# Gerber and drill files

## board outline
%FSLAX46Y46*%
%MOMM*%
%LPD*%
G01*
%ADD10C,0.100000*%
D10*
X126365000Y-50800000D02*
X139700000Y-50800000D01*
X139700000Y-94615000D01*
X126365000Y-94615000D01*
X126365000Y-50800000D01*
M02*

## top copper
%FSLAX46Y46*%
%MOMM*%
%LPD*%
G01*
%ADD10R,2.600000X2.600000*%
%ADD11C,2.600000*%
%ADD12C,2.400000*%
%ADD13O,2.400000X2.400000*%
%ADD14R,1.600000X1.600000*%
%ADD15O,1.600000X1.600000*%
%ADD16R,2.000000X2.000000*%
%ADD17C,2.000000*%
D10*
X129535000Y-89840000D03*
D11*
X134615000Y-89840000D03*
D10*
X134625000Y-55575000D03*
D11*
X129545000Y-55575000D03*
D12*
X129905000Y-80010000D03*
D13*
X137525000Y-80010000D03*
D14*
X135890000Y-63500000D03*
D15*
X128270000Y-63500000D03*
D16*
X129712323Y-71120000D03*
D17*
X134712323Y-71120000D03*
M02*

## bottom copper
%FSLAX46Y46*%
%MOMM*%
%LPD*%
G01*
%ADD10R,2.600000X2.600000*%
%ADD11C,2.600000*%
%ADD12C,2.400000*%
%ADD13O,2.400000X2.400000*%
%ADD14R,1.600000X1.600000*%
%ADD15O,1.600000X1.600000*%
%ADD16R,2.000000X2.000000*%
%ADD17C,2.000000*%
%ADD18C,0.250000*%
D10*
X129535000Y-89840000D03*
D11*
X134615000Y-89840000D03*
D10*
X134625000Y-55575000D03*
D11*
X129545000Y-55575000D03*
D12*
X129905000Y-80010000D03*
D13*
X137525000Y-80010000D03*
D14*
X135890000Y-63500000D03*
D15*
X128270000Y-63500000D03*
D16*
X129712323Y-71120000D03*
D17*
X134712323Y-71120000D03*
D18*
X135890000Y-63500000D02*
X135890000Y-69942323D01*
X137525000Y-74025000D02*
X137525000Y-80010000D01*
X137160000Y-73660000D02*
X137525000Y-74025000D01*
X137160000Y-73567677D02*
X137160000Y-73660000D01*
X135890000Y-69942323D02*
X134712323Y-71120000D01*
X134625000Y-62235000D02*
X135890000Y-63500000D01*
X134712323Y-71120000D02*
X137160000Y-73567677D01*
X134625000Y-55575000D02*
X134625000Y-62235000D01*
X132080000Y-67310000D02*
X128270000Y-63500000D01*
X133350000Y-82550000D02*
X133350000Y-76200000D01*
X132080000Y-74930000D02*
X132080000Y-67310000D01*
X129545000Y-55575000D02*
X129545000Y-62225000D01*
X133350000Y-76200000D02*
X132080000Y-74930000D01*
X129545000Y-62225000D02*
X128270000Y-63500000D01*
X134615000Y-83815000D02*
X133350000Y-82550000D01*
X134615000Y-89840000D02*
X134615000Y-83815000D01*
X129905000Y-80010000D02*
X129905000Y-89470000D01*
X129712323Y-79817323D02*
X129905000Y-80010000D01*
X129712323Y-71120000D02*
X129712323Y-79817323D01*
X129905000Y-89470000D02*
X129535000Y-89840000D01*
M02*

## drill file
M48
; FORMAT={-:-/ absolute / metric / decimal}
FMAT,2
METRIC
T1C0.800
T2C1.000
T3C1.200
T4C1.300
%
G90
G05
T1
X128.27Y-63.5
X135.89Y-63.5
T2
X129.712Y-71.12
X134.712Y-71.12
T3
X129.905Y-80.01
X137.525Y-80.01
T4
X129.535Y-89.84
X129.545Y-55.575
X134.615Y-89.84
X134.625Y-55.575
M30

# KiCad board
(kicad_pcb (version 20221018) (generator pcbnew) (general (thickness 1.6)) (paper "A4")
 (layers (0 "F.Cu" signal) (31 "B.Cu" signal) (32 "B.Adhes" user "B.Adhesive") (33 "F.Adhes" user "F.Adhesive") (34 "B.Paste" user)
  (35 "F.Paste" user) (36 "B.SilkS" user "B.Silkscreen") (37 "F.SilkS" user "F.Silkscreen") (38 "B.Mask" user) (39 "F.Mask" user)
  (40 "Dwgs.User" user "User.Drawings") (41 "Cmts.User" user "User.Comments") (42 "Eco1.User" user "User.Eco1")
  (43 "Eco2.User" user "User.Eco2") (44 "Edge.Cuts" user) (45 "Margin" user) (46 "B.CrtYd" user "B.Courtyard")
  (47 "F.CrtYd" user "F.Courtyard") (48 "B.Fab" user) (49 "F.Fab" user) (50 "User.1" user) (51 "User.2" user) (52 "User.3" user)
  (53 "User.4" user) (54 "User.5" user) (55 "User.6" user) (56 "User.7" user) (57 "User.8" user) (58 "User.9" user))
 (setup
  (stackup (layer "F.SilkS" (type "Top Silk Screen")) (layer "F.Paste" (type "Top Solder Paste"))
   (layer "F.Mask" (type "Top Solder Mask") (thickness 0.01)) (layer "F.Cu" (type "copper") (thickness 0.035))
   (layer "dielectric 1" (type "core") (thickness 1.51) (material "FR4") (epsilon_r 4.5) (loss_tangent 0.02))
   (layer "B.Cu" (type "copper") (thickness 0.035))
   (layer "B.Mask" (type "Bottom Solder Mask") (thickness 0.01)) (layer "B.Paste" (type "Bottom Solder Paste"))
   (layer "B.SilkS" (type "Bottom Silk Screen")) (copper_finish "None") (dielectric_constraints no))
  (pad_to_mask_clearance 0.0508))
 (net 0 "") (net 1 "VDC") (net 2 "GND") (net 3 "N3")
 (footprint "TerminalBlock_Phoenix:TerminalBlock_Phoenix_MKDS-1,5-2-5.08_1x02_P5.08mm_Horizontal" (layer "F.Cu") (at 129.535 89.84)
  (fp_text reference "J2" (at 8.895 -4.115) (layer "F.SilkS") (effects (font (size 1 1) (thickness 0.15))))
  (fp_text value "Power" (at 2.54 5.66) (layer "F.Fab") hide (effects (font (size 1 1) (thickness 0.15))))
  (pad "1" thru_hole rect (at 0 0) (size 2.6 2.6) (drill 1.3) (layers "*.Cu" "*.Mask") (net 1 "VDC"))
  (pad "2" thru_hole circle (at 5.08 0) (size 2.6 2.6) (drill 1.3) (layers "*.Cu" "*.Mask") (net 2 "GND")))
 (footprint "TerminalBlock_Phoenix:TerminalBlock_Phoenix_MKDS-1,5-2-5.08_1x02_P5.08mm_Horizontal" (layer "F.Cu") (at 134.625 55.575 180)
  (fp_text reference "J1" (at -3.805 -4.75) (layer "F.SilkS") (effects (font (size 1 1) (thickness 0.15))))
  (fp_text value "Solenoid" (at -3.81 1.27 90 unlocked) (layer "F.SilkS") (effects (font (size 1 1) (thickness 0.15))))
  (pad "1" thru_hole rect (at 0 0 180) (size 2.6 2.6) (drill 1.3) (layers "*.Cu" "*.Mask") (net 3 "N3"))
  (pad "2" thru_hole circle (at 5.08 0 180) (size 2.6 2.6) (drill 1.3) (layers "*.Cu" "*.Mask") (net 2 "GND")))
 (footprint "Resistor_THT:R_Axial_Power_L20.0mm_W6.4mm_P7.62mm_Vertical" (layer "F.Cu") (at 129.905 80.01)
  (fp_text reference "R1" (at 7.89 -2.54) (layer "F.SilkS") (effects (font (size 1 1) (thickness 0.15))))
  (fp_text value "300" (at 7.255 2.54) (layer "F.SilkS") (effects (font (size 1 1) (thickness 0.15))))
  (pad "1" thru_hole circle (at 0 0) (size 2.4 2.4) (drill 1.2) (layers "*.Cu" "*.Mask") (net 1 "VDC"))
  (pad "2" thru_hole oval (at 7.62 0) (size 2.4 2.4) (drill 1.2) (layers "*.Cu" "*.Mask") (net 3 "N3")))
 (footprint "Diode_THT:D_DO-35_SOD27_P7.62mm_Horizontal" (layer "F.Cu") (at 135.89 63.5 180)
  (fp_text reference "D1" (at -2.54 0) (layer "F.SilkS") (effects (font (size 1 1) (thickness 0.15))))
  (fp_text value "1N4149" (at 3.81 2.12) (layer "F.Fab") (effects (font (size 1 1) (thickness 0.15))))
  (pad "1" thru_hole rect (at 0 0 180) (size 1.6 1.6) (drill 0.8) (layers "*.Cu" "*.Mask") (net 3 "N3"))
  (pad "2" thru_hole oval (at 7.62 0 180) (size 1.6 1.6) (drill 0.8) (layers "*.Cu" "*.Mask") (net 2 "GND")))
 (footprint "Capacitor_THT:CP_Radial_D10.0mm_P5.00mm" (layer "F.Cu") (at 129.712323 71.12)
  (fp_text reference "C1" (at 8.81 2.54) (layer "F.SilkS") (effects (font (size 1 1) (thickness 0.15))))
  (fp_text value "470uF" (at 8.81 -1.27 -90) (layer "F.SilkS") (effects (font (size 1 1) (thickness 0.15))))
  (pad "1" thru_hole rect (at 0 0) (size 2 2) (drill 1) (layers "*.Cu" "*.Mask") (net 1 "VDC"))
  (pad "2" thru_hole circle (at 5 0) (size 2 2) (drill 1) (layers "*.Cu" "*.Mask") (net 3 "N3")))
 (gr_rect (start 126.365 50.8) (end 139.7 94.615) (stroke (width 0.1) (type default)) (fill none) (layer "Edge.Cuts"))
 (segment (start 135.89 63.5) (end 135.89 69.942323) (width 0.25) (layer "B.Cu") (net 3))
 (segment (start 137.525 74.025) (end 137.525 80.01) (width 0.25) (layer "B.Cu") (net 3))
 (segment (start 137.16 73.66) (end 137.525 74.025) (width 0.25) (layer "B.Cu") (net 3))
 (segment (start 137.16 73.567677) (end 137.16 73.66) (width 0.25) (layer "B.Cu") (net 3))
 (segment (start 135.89 69.942323) (end 134.712323 71.12) (width 0.25) (layer "B.Cu") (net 3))
 (segment (start 134.625 62.235) (end 135.89 63.5) (width 0.25) (layer "B.Cu") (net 3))
 (segment (start 134.712323 71.12) (end 137.16 73.567677) (width 0.25) (layer "B.Cu") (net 3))
 (segment (start 134.625 55.575) (end 134.625 62.235) (width 0.25) (layer "B.Cu") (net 3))
 (segment (start 132.08 67.31) (end 128.27 63.5) (width 0.25) (layer "B.Cu") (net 2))
 (segment (start 133.35 82.55) (end 133.35 76.2) (width 0.25) (layer "B.Cu") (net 2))
 (segment (start 132.08 74.93) (end 132.08 67.31) (width 0.25) (layer "B.Cu") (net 2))
 (segment (start 129.545 55.575) (end 129.545 62.225) (width 0.25) (layer "B.Cu") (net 2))
 (segment (start 133.35 76.2) (end 132.08 74.93) (width 0.25) (layer "B.Cu") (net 2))
 (segment (start 129.545 62.225) (end 128.27 63.5) (width 0.25) (layer "B.Cu") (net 2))
 (segment (start 134.615 83.815) (end 133.35 82.55) (width 0.25) (layer "B.Cu") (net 2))
 (segment (start 134.615 89.84) (end 134.615 83.815) (width 0.25) (layer "B.Cu") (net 2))
 (segment (start 129.905 80.01) (end 129.905 89.47) (width 0.25) (layer "B.Cu") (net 1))
 (segment (start 129.712323 79.817323) (end 129.905 80.01) (width 0.25) (layer "B.Cu") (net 1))
 (segment (start 129.712323 71.12) (end 129.712323 79.817323) (width 0.25) (layer "B.Cu") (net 1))
 (segment (start 129.905 89.47) (end 129.535 89.84) (width 0.25) (layer "B.Cu") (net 1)))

